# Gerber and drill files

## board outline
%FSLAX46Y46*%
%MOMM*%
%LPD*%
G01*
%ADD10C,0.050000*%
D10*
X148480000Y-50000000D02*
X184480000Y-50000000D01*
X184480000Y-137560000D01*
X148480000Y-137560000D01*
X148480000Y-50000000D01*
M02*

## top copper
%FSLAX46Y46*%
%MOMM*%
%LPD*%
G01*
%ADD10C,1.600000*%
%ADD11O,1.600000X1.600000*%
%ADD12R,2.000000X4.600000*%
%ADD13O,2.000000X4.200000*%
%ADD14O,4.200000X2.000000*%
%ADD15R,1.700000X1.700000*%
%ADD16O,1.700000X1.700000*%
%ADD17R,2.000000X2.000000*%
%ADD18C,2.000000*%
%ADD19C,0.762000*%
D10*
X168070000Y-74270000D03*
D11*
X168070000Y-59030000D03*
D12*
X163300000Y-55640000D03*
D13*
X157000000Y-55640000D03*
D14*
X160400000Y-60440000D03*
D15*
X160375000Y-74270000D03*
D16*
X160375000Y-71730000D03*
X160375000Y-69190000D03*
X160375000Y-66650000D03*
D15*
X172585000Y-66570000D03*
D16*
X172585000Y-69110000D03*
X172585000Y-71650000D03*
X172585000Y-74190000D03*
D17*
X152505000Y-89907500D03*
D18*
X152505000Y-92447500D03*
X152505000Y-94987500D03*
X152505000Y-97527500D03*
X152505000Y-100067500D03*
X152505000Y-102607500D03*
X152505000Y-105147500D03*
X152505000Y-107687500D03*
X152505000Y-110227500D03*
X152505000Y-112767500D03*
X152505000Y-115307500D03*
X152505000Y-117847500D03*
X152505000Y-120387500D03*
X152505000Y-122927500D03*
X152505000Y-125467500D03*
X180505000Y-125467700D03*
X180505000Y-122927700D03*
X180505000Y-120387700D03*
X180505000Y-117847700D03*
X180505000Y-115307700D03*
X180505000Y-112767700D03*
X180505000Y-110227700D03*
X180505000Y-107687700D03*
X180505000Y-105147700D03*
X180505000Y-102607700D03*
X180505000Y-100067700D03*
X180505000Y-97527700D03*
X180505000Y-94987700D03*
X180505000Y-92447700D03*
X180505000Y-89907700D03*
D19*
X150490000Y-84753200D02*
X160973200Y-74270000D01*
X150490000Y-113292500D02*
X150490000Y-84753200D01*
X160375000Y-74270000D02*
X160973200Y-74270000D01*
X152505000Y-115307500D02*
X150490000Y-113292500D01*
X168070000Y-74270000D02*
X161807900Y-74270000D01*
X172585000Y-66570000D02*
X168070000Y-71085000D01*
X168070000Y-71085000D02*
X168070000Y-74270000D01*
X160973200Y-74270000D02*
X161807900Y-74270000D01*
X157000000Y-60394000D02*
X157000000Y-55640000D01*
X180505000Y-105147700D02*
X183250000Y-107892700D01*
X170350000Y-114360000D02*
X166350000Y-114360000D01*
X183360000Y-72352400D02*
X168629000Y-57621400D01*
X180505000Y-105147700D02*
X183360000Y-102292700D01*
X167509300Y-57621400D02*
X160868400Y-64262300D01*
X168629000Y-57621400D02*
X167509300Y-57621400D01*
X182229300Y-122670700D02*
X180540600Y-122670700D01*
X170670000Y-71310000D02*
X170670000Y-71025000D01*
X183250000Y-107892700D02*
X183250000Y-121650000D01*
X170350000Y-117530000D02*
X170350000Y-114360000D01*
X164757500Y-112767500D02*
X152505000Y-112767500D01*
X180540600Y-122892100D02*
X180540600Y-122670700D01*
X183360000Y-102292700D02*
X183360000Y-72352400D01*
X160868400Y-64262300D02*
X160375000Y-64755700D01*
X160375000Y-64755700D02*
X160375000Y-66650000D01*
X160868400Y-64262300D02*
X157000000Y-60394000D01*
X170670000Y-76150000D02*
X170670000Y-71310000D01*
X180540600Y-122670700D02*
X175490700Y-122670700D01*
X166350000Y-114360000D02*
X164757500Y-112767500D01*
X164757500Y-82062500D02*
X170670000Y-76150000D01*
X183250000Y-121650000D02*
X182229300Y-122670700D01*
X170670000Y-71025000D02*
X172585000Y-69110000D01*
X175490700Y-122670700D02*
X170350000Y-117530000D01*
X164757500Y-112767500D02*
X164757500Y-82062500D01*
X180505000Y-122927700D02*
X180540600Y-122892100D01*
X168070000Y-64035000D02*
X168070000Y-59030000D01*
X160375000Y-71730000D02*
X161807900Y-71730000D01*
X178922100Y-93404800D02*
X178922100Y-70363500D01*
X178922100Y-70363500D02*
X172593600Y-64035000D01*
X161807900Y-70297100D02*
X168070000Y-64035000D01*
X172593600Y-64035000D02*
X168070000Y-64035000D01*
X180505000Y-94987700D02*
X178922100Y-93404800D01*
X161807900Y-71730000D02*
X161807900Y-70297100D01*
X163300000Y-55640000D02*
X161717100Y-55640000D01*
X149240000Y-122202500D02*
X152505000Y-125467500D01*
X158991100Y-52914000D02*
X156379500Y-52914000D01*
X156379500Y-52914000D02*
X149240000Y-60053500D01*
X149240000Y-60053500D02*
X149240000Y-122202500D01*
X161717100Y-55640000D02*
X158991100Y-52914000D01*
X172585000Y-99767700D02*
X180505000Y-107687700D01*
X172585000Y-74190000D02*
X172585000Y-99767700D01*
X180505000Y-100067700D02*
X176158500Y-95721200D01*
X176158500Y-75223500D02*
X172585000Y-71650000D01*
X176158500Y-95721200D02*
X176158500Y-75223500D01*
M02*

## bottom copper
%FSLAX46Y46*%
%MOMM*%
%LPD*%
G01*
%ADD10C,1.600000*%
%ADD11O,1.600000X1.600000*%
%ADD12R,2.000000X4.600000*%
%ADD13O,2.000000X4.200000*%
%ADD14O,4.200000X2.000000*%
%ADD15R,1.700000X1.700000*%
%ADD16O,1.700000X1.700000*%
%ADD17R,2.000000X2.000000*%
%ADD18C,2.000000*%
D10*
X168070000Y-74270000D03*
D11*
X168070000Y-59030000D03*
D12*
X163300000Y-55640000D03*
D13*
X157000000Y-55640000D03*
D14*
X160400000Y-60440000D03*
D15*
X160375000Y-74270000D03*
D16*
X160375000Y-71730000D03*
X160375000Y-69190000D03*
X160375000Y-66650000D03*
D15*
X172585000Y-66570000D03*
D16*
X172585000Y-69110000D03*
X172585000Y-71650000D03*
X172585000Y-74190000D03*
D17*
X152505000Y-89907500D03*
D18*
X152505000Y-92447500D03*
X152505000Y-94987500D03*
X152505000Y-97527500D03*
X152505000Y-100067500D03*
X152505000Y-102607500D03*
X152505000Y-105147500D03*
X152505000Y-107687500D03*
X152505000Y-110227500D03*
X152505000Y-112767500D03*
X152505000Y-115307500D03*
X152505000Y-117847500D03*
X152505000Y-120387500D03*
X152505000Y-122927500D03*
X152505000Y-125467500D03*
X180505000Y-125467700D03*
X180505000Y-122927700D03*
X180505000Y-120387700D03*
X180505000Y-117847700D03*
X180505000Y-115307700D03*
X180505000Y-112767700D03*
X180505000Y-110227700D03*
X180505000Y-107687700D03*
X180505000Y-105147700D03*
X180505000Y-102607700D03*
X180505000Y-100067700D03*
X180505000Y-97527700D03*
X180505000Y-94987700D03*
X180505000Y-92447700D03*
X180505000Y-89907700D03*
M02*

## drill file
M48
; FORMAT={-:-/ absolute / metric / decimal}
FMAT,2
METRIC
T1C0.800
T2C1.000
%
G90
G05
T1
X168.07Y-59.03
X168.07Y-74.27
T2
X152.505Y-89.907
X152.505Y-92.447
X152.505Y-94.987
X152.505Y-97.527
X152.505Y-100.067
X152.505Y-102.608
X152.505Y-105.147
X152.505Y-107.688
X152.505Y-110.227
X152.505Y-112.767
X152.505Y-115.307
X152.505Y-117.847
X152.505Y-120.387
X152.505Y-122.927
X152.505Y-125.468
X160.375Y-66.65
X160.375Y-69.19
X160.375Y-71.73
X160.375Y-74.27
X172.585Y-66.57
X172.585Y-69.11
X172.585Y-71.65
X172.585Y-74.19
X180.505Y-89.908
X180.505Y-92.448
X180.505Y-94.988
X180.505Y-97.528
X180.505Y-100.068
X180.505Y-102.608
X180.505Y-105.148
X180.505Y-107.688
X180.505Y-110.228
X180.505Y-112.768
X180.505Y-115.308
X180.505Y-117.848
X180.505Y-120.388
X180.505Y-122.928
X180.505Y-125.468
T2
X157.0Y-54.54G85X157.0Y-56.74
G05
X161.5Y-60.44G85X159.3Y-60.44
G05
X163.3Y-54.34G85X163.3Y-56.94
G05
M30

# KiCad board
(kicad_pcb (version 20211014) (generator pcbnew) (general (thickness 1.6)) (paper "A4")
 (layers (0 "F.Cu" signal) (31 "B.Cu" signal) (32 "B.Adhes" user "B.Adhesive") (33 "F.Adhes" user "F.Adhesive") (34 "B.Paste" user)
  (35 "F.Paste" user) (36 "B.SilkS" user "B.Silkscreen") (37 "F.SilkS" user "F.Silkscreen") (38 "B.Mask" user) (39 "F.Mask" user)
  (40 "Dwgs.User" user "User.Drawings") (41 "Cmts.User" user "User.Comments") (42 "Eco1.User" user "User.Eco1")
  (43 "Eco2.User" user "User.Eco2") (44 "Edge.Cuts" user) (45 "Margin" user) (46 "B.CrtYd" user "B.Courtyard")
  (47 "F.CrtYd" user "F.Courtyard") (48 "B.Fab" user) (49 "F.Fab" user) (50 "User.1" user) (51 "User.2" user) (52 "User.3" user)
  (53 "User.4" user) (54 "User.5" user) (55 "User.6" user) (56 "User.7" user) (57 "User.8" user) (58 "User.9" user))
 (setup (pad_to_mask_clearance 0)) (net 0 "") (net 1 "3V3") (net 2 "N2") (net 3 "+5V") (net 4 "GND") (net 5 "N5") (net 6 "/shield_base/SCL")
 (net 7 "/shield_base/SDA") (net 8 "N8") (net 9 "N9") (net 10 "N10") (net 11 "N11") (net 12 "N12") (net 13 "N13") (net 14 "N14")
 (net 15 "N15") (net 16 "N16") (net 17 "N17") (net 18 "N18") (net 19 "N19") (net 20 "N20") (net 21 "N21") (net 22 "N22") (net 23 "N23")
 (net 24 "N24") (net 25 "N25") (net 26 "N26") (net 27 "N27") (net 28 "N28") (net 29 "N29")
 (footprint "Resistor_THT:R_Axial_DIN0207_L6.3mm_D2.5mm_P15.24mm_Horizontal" (layer "F.Cu") (at 168.07 74.27 90)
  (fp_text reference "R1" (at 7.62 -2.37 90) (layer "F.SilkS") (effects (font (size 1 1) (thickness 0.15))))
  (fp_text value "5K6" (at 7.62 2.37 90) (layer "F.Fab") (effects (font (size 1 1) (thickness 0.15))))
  (pad "1" thru_hole circle (at 0 0 90) (size 1.6 1.6) (drill 0.8) (layers *.Cu *.Mask) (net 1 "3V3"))
  (pad "2" thru_hole oval (at 15.24 0 90) (size 1.6 1.6) (drill 0.8) (layers *.Cu *.Mask) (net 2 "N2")))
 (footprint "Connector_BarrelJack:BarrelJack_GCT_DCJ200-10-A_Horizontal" (layer "F.Cu") (at 163.3 55.64 -90)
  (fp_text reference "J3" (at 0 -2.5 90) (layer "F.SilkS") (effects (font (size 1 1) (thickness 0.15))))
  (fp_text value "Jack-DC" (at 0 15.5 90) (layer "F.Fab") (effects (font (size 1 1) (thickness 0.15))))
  (pad "1" thru_hole rect (at 0 0 270) (size 4.6 2) (drill oval 3.6 1) (layers *.Cu *.Mask) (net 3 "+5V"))
  (pad "2" thru_hole oval (at 0 6.3 270) (size 4.2 2) (drill oval 3.2 1) (layers *.Cu *.Mask) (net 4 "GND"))
  (pad "3" thru_hole oval (at 4.8 2.9 270) (size 2 4.2) (drill oval 1 3.2) (layers *.Cu *.Mask)))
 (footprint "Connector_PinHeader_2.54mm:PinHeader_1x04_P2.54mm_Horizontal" (layer "F.Cu") (at 160.375 74.27 180)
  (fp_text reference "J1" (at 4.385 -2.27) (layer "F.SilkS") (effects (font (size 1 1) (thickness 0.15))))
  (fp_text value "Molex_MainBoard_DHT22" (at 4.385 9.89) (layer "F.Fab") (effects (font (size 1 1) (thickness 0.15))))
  (pad "1" thru_hole rect (at 0 0 180) (size 1.7 1.7) (drill 1) (layers *.Cu *.Mask) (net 1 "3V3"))
  (pad "2" thru_hole oval (at 0 2.54 180) (size 1.7 1.7) (drill 1) (layers *.Cu *.Mask) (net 2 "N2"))
  (pad "3" thru_hole oval (at 0 5.08 180) (size 1.7 1.7) (drill 1) (layers *.Cu *.Mask) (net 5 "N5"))
  (pad "4" thru_hole oval (at 0 7.62 180) (size 1.7 1.7) (drill 1) (layers *.Cu *.Mask) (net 4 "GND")))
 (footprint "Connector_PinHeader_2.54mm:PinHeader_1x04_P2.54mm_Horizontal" (layer "F.Cu") (at 172.585 66.57)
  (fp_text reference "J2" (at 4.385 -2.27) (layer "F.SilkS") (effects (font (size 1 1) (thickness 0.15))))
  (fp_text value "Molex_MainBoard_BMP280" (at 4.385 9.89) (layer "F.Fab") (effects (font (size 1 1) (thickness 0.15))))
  (pad "1" thru_hole rect (at 0 0) (size 1.7 1.7) (drill 1) (layers *.Cu *.Mask) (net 1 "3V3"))
  (pad "2" thru_hole oval (at 0 2.54) (size 1.7 1.7) (drill 1) (layers *.Cu *.Mask) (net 4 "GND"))
  (pad "3" thru_hole oval (at 0 5.08) (size 1.7 1.7) (drill 1) (layers *.Cu *.Mask) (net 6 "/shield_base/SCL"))
  (pad "4" thru_hole oval (at 0 7.62) (size 1.7 1.7) (drill 1) (layers *.Cu *.Mask) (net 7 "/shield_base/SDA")))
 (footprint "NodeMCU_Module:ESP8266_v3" (layer "F.Cu") (at 164.855 140.9675)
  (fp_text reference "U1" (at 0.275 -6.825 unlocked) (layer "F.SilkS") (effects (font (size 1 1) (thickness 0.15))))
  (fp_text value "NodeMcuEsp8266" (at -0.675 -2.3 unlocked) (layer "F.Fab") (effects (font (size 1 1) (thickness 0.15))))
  (pad "1" thru_hole rect (at -12.35 -51.06 180) (size 2 2) (drill 1) (layers *.Cu *.Mask) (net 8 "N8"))
  (pad "2" thru_hole circle (at -12.35 -48.52 180) (size 2 2) (drill 1) (layers *.Cu *.Mask) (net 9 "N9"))
  (pad "3" thru_hole circle (at -12.35 -45.98 180) (size 2 2) (drill 1) (layers *.Cu *.Mask) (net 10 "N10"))
  (pad "4" thru_hole circle (at -12.35 -43.44 180) (size 2 2) (drill 1) (layers *.Cu *.Mask) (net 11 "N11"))
  (pad "5" thru_hole circle (at -12.35 -40.9 180) (size 2 2) (drill 1) (layers *.Cu *.Mask) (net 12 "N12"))
  (pad "6" thru_hole circle (at -12.35 -38.36 180) (size 2 2) (drill 1) (layers *.Cu *.Mask) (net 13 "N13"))
  (pad "7" thru_hole circle (at -12.35 -35.82 180) (size 2 2) (drill 1) (layers *.Cu *.Mask) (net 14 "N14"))
  (pad "8" thru_hole circle (at -12.35 -33.28 180) (size 2 2) (drill 1) (layers *.Cu *.Mask) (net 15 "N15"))
  (pad "9" thru_hole circle (at -12.35 -30.74 180) (size 2 2) (drill 1) (layers *.Cu *.Mask) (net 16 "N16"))
  (pad "10" thru_hole circle (at -12.35 -28.2 180) (size 2 2) (drill 1) (layers *.Cu *.Mask) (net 4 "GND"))
  (pad "11" thru_hole circle (at -12.35 -25.66 180) (size 2 2) (drill 1) (layers *.Cu *.Mask) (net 1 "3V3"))
  (pad "12" thru_hole circle (at -12.35 -23.12 180) (size 2 2) (drill 1) (layers *.Cu *.Mask) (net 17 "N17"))
  (pad "13" thru_hole circle (at -12.35 -20.58 180) (size 2 2) (drill 1) (layers *.Cu *.Mask) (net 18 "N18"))
  (pad "14" thru_hole circle (at -12.35 -18.04 180) (size 2 2) (drill 1) (layers *.Cu *.Mask) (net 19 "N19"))
  (pad "15" thru_hole circle (at -12.35 -15.5 90) (size 2 2) (drill 1) (layers *.Cu *.Mask) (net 3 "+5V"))
  (pad "16" thru_hole circle (at 15.65 -15.4998 180) (size 2 2) (drill 1) (layers *.Cu *.Mask) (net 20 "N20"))
  (pad "17" thru_hole circle (at 15.65 -18.0398 180) (size 2 2) (drill 1) (layers *.Cu *.Mask) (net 4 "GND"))
  (pad "18" thru_hole circle (at 15.65 -20.5798 180) (size 2 2) (drill 1) (layers *.Cu *.Mask) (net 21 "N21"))
  (pad "19" thru_hole circle (at 15.65 -23.1198 180) (size 2 2) (drill 1) (layers *.Cu *.Mask) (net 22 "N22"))
  (pad "20" thru_hole circle (at 15.65 -25.6598 180) (size 2 2) (drill 1) (layers *.Cu *.Mask) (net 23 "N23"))
  (pad "21" thru_hole circle (at 15.65 -28.1998 180) (size 2 2) (drill 1) (layers *.Cu *.Mask) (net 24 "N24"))
  (pad "22" thru_hole circle (at 15.65 -30.7398 180) (size 2 2) (drill 1) (layers *.Cu *.Mask) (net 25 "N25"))
  (pad "23" thru_hole circle (at 15.65 -33.2798 180) (size 2 2) (drill 1) (layers *.Cu *.Mask) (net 7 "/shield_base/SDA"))
  (pad "24" thru_hole circle (at 15.65 -35.8198 180) (size 2 2) (drill 1) (layers *.Cu *.Mask) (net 4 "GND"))
  (pad "25" thru_hole circle (at 15.65 -38.3598 180) (size 2 2) (drill 1) (layers *.Cu *.Mask) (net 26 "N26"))
  (pad "26" thru_hole circle (at 15.65 -40.8998 180) (size 2 2) (drill 1) (layers *.Cu *.Mask) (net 6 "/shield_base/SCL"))
  (pad "27" thru_hole circle (at 15.65 -43.4398 180) (size 2 2) (drill 1) (layers *.Cu *.Mask) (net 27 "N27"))
  (pad "28" thru_hole circle (at 15.65 -45.9798 180) (size 2 2) (drill 1) (layers *.Cu *.Mask) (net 2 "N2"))
  (pad "29" thru_hole circle (at 15.65 -48.5198 180) (size 2 2) (drill 1) (layers *.Cu *.Mask) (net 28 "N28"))
  (pad "30" thru_hole circle (at 15.65 -51.0598 180) (size 2 2) (drill 1) (layers *.Cu *.Mask) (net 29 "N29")))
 (gr_rect (start 148.48 50) (end 184.48 137.56) (layer "Edge.Cuts") (width 0.05) (fill none))
 (segment (start 150.49 84.7532) (end 160.9732 74.27) (width 0.762) (layer "F.Cu") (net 1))
 (segment (start 150.49 113.2925) (end 150.49 84.7532) (width 0.762) (layer "F.Cu") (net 1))
 (segment (start 160.375 74.27) (end 160.9732 74.27) (width 0.762) (layer "F.Cu") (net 1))
 (segment (start 152.505 115.3075) (end 150.49 113.2925) (width 0.762) (layer "F.Cu") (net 1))
 (segment (start 168.07 74.27) (end 161.8079 74.27) (width 0.762) (layer "F.Cu") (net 1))
 (segment (start 172.585 66.57) (end 168.07 71.085) (width 0.762) (layer "F.Cu") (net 1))
 (segment (start 168.07 71.085) (end 168.07 74.27) (width 0.762) (layer "F.Cu") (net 1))
 (segment (start 160.9732 74.27) (end 161.8079 74.27) (width 0.762) (layer "F.Cu") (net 1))
 (segment (start 157 60.394) (end 157 55.64) (width 0.762) (layer "F.Cu") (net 4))
 (segment (start 180.505 105.1477) (end 183.25 107.8927) (width 0.762) (layer "F.Cu") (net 4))
 (segment (start 170.35 114.36) (end 166.35 114.36) (width 0.762) (layer "F.Cu") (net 4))
 (segment (start 183.36 72.3524) (end 168.629 57.6214) (width 0.762) (layer "F.Cu") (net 4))
 (segment (start 180.505 105.1477) (end 183.36 102.2927) (width 0.762) (layer "F.Cu") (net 4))
 (segment (start 167.5093 57.6214) (end 160.8684 64.2623) (width 0.762) (layer "F.Cu") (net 4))
 (segment (start 168.629 57.6214) (end 167.5093 57.6214) (width 0.762) (layer "F.Cu") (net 4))
 (segment (start 182.2293 122.6707) (end 180.5406 122.6707) (width 0.762) (layer "F.Cu") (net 4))
 (segment (start 170.67 71.31) (end 170.67 71.025) (width 0.762) (layer "F.Cu") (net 4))
 (segment (start 183.25 107.8927) (end 183.25 121.65) (width 0.762) (layer "F.Cu") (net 4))
 (segment (start 170.35 117.53) (end 170.35 114.36) (width 0.762) (layer "F.Cu") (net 4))
 (segment (start 164.7575 112.7675) (end 152.505 112.7675) (width 0.762) (layer "F.Cu") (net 4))
 (segment (start 180.5406 122.8921) (end 180.5406 122.6707) (width 0.762) (layer "F.Cu") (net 4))
 (segment (start 183.36 102.2927) (end 183.36 72.3524) (width 0.762) (layer "F.Cu") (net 4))
 (segment (start 160.8684 64.2623) (end 160.375 64.7557) (width 0.762) (layer "F.Cu") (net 4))
 (segment (start 160.375 64.7557) (end 160.375 66.65) (width 0.762) (layer "F.Cu") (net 4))
 (segment (start 160.8684 64.2623) (end 157 60.394) (width 0.762) (layer "F.Cu") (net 4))
 (segment (start 170.67 76.15) (end 170.67 71.31) (width 0.762) (layer "F.Cu") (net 4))
 (segment (start 180.5406 122.6707) (end 175.4907 122.6707) (width 0.762) (layer "F.Cu") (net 4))
 (segment (start 166.35 114.36) (end 164.7575 112.7675) (width 0.762) (layer "F.Cu") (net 4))
 (segment (start 164.7575 82.0625) (end 170.67 76.15) (width 0.762) (layer "F.Cu") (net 4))
 (segment (start 183.25 121.65) (end 182.2293 122.6707) (width 0.762) (layer "F.Cu") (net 4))
 (segment (start 170.67 71.025) (end 172.585 69.11) (width 0.762) (layer "F.Cu") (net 4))
 (segment (start 175.4907 122.6707) (end 170.35 117.53) (width 0.762) (layer "F.Cu") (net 4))
 (segment (start 164.7575 112.7675) (end 164.7575 82.0625) (width 0.762) (layer "F.Cu") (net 4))
 (segment (start 180.505 122.9277) (end 180.5406 122.8921) (width 0.762) (layer "F.Cu") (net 4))
 (segment (start 168.07 64.035) (end 168.07 59.03) (width 0.762) (layer "F.Cu") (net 2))
 (segment (start 160.375 71.73) (end 161.8079 71.73) (width 0.762) (layer "F.Cu") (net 2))
 (segment (start 178.9221 93.4048) (end 178.9221 70.3635) (width 0.762) (layer "F.Cu") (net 2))
 (segment (start 178.9221 70.3635) (end 172.5936 64.035) (width 0.762) (layer "F.Cu") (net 2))
 (segment (start 161.8079 70.2971) (end 168.07 64.035) (width 0.762) (layer "F.Cu") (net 2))
 (segment (start 172.5936 64.035) (end 168.07 64.035) (width 0.762) (layer "F.Cu") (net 2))
 (segment (start 180.505 94.9877) (end 178.9221 93.4048) (width 0.762) (layer "F.Cu") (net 2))
 (segment (start 161.8079 71.73) (end 161.8079 70.2971) (width 0.762) (layer "F.Cu") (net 2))
 (segment (start 163.3 55.64) (end 161.7171 55.64) (width 0.762) (layer "F.Cu") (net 3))
 (segment (start 149.24 122.2025) (end 152.505 125.4675) (width 0.762) (layer "F.Cu") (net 3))
 (segment (start 158.9911 52.914) (end 156.3795 52.914) (width 0.762) (layer "F.Cu") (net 3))
 (segment (start 156.3795 52.914) (end 149.24 60.0535) (width 0.762) (layer "F.Cu") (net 3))
 (segment (start 149.24 60.0535) (end 149.24 122.2025) (width 0.762) (layer "F.Cu") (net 3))
 (segment (start 161.7171 55.64) (end 158.9911 52.914) (width 0.762) (layer "F.Cu") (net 3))
 (segment (start 172.585 99.7677) (end 180.505 107.6877) (width 0.762) (layer "F.Cu") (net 7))
 (segment (start 172.585 74.19) (end 172.585 99.7677) (width 0.762) (layer "F.Cu") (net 7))
 (segment (start 180.505 100.0677) (end 176.1585 95.7212) (width 0.762) (layer "F.Cu") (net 6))
 (segment (start 176.1585 75.2235) (end 172.585 71.65) (width 0.762) (layer "F.Cu") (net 6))
 (segment (start 176.1585 95.7212) (end 176.1585 75.2235) (width 0.762) (layer "F.Cu") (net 6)))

